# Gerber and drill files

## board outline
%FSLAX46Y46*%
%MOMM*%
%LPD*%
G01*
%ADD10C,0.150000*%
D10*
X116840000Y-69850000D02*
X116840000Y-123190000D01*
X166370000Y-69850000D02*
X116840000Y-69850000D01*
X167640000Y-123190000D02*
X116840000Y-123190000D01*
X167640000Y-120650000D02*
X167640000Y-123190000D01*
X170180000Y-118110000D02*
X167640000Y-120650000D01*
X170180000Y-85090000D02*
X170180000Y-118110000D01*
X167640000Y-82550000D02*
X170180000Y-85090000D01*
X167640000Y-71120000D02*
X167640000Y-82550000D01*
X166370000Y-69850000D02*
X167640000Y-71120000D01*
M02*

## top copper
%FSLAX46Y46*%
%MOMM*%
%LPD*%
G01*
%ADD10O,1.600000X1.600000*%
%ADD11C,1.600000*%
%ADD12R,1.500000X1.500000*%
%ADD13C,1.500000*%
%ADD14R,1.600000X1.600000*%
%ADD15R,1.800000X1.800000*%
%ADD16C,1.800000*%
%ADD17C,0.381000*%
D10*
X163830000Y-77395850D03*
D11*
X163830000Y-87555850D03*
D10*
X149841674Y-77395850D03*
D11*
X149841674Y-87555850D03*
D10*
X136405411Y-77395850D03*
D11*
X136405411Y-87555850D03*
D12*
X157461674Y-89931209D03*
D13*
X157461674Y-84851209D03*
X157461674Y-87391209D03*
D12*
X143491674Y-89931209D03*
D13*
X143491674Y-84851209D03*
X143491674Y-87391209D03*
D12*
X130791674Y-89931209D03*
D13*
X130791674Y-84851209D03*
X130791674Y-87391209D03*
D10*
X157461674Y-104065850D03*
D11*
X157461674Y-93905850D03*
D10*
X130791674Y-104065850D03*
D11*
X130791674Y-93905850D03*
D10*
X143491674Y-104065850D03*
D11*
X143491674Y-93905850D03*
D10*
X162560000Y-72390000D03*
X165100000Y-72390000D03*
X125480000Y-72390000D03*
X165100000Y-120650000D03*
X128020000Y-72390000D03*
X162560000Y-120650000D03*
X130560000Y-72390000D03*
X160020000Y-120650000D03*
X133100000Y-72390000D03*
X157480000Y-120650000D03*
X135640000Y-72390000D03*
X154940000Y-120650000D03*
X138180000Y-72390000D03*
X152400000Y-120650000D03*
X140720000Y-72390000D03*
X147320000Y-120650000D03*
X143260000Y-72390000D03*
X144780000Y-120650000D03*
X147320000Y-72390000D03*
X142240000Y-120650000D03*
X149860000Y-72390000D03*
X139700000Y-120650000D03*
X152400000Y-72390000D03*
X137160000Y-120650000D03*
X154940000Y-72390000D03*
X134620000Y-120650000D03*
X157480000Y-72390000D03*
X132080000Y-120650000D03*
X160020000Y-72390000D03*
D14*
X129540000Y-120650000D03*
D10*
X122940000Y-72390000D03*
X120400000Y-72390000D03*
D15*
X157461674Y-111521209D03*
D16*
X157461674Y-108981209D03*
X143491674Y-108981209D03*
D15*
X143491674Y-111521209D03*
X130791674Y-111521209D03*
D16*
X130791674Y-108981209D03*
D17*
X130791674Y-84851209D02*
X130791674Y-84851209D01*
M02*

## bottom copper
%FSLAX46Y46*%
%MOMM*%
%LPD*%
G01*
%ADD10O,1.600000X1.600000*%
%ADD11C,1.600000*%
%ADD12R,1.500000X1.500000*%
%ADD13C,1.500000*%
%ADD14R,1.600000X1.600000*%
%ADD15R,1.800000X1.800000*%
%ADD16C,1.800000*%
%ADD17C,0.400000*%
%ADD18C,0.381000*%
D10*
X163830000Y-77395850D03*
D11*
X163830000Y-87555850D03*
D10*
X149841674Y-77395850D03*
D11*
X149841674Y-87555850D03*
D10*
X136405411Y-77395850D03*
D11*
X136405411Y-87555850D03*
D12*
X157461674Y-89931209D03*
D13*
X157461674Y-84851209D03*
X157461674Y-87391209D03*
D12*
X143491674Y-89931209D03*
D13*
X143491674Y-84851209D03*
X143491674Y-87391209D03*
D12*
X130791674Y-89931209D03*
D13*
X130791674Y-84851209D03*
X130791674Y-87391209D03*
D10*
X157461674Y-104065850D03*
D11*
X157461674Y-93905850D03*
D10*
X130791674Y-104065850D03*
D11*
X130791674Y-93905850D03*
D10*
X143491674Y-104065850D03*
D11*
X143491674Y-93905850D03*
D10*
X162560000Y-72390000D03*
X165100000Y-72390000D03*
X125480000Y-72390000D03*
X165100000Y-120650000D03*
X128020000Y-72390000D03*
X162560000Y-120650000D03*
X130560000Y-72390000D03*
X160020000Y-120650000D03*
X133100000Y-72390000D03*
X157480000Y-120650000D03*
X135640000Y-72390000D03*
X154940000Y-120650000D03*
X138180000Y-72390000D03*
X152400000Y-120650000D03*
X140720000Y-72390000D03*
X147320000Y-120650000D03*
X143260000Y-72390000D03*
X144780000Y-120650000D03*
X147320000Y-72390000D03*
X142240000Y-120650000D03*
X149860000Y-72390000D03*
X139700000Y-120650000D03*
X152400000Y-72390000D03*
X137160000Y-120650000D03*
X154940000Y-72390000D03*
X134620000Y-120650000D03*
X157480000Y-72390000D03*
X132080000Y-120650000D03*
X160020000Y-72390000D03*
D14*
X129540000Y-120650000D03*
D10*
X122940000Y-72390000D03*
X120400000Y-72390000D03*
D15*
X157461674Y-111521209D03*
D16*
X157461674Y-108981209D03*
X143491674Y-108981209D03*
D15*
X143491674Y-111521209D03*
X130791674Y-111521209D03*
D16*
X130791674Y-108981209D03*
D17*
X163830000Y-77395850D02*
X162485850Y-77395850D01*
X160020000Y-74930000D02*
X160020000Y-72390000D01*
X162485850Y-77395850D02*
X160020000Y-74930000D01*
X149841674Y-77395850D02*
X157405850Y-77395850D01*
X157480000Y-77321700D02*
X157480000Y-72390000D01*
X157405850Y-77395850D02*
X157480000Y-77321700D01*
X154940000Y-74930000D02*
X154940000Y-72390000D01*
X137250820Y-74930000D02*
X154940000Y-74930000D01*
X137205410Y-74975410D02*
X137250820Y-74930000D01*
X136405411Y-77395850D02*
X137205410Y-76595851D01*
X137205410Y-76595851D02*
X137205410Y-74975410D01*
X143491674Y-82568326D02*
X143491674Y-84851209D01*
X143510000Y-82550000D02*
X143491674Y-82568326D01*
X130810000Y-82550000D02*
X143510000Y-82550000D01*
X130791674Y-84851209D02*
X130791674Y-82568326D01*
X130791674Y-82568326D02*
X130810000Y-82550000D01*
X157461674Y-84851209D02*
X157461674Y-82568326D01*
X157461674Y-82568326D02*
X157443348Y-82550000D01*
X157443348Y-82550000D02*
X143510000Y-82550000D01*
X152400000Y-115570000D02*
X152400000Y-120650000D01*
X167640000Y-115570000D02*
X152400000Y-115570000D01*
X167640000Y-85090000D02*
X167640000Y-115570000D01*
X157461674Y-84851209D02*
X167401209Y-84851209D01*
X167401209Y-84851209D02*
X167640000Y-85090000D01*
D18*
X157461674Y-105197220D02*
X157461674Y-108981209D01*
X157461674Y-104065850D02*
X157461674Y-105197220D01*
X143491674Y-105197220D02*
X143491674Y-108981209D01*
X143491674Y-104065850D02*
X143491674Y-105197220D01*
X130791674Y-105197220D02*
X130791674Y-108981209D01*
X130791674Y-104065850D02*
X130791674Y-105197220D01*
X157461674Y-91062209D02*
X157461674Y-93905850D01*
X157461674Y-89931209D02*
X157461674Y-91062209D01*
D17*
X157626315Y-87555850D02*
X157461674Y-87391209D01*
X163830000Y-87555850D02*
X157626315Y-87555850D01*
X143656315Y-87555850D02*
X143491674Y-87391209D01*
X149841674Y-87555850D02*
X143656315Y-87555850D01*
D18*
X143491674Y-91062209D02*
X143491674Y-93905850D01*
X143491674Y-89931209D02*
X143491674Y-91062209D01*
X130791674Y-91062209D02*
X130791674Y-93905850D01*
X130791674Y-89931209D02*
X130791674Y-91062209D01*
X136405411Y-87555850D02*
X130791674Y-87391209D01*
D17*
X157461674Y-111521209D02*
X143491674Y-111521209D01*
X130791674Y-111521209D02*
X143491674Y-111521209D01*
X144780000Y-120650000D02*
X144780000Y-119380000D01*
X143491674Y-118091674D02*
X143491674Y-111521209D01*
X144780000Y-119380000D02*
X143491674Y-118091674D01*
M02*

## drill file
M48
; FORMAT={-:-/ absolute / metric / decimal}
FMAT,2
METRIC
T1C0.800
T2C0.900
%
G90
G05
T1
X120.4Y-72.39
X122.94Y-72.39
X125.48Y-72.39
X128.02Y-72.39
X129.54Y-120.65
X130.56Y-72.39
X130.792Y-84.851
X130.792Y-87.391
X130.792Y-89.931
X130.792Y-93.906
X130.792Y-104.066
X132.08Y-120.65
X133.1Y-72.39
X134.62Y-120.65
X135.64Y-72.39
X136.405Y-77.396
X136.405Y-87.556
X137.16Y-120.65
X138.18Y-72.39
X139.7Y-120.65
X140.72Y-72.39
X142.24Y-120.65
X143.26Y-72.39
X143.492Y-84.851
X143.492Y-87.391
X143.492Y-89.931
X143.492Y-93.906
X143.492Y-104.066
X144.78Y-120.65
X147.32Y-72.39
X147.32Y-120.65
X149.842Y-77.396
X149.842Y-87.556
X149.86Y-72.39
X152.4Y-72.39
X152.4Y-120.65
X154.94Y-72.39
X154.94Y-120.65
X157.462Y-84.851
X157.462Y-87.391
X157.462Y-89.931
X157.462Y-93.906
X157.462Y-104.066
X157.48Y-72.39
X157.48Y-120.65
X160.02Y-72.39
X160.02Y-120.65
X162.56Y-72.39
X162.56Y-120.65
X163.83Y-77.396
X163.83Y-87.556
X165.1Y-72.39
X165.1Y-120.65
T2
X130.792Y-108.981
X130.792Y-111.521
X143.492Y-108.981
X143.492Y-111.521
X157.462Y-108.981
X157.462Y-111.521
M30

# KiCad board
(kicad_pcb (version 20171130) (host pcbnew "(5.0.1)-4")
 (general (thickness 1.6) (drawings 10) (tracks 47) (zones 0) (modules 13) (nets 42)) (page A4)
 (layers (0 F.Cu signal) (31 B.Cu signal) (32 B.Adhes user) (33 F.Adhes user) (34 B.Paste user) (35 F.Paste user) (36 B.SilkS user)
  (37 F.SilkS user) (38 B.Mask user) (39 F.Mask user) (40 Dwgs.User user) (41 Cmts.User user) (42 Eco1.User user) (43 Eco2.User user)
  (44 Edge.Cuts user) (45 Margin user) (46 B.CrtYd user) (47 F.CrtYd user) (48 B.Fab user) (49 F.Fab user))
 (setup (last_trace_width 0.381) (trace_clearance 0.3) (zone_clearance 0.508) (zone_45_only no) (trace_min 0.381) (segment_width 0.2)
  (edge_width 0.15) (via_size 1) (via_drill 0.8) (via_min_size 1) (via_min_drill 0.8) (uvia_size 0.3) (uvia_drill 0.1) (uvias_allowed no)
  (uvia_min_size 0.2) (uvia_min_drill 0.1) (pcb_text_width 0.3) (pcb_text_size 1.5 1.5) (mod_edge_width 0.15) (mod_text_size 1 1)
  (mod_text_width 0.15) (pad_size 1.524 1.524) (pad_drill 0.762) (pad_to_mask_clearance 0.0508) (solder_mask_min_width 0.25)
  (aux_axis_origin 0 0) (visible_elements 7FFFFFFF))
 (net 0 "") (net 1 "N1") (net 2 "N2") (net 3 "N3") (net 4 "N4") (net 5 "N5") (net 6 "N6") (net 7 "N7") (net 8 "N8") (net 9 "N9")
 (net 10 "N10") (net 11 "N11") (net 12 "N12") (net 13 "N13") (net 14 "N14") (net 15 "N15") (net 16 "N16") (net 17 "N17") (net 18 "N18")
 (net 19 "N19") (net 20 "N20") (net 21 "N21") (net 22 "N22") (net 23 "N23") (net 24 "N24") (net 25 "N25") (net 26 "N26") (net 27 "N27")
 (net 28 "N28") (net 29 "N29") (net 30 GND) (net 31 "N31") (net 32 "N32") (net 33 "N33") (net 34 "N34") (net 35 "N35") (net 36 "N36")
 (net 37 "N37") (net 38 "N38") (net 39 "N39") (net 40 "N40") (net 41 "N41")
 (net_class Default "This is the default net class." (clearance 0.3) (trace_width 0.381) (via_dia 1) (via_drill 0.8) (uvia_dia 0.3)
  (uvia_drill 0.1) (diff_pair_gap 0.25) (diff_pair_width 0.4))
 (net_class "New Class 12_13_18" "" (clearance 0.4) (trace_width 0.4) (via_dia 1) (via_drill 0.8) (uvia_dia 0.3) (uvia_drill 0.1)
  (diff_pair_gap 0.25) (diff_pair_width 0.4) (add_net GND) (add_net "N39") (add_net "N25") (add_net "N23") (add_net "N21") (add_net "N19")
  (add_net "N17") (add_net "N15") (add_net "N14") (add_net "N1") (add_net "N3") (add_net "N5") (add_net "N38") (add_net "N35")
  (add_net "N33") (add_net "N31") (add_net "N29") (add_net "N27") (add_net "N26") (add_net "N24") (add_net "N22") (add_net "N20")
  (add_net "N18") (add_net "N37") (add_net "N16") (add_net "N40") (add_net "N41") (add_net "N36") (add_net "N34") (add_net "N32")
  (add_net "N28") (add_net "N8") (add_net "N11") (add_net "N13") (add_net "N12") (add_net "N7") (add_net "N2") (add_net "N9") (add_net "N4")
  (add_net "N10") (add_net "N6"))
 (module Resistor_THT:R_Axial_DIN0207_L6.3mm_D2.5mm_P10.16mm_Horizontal (layer F.Cu) (at 163.83 87.55585 90)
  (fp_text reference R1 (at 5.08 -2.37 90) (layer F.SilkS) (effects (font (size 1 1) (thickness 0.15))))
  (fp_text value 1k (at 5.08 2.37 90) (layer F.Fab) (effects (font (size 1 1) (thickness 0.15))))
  (pad 2 thru_hole oval (at 10.16 0 90) (size 1.6 1.6) (drill 0.8) (layers *.Cu *.Mask) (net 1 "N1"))
  (pad 1 thru_hole circle (at 0 0 90) (size 1.6 1.6) (drill 0.8) (layers *.Cu *.Mask) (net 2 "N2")))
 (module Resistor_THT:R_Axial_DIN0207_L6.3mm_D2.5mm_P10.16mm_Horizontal (layer F.Cu) (at 149.841674 87.55585 90)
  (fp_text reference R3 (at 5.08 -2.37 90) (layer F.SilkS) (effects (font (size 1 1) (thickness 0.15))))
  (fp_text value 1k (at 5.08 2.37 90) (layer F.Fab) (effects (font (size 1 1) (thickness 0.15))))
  (pad 2 thru_hole oval (at 10.16 0 90) (size 1.6 1.6) (drill 0.8) (layers *.Cu *.Mask) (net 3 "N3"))
  (pad 1 thru_hole circle (at 0 0 90) (size 1.6 1.6) (drill 0.8) (layers *.Cu *.Mask) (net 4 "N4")))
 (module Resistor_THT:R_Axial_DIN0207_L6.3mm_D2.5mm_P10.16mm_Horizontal (layer F.Cu) (at 136.405411 87.55585 90)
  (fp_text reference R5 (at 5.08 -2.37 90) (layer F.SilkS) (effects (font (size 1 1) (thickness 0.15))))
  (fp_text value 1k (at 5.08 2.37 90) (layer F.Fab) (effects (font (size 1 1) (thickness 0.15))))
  (pad 2 thru_hole oval (at 10.16 0 90) (size 1.6 1.6) (drill 0.8) (layers *.Cu *.Mask) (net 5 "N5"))
  (pad 1 thru_hole circle (at 0 0 90) (size 1.6 1.6) (drill 0.8) (layers *.Cu *.Mask) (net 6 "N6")))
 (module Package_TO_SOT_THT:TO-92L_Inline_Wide (layer F.Cu) (at 157.461674 89.931209 90)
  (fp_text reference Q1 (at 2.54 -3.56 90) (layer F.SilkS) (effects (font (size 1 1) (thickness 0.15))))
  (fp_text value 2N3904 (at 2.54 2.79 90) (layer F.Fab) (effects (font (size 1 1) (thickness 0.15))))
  (pad 1 thru_hole rect (at 0 0 180) (size 1.5 1.5) (drill 0.8) (layers *.Cu *.Mask) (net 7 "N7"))
  (pad 3 thru_hole circle (at 5.08 0 180) (size 1.5 1.5) (drill 0.8) (layers *.Cu *.Mask) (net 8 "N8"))
  (pad 2 thru_hole circle (at 2.54 0 180) (size 1.5 1.5) (drill 0.8) (layers *.Cu *.Mask) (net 2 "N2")))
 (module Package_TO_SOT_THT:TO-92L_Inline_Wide (layer F.Cu) (at 143.491674 89.931209 90)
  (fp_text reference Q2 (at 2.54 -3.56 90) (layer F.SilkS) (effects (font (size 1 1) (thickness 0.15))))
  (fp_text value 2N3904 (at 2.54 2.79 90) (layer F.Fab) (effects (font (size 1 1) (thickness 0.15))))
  (pad 1 thru_hole rect (at 0 0 180) (size 1.5 1.5) (drill 0.8) (layers *.Cu *.Mask) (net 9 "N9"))
  (pad 3 thru_hole circle (at 5.08 0 180) (size 1.5 1.5) (drill 0.8) (layers *.Cu *.Mask) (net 8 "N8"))
  (pad 2 thru_hole circle (at 2.54 0 180) (size 1.5 1.5) (drill 0.8) (layers *.Cu *.Mask) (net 4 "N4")))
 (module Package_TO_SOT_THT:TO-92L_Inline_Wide (layer F.Cu) (at 130.791674 89.931209 90)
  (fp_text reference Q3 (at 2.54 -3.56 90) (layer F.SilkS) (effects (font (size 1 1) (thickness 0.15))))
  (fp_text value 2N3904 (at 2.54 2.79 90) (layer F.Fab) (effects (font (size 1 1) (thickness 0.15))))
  (pad 1 thru_hole rect (at 0 0 180) (size 1.5 1.5) (drill 0.8) (layers *.Cu *.Mask) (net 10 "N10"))
  (pad 3 thru_hole circle (at 5.08 0 180) (size 1.5 1.5) (drill 0.8) (layers *.Cu *.Mask) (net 8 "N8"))
  (pad 2 thru_hole circle (at 2.54 0 180) (size 1.5 1.5) (drill 0.8) (layers *.Cu *.Mask) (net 6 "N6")))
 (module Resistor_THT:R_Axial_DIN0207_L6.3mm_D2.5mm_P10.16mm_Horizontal (layer F.Cu) (at 157.461674 93.90585 270)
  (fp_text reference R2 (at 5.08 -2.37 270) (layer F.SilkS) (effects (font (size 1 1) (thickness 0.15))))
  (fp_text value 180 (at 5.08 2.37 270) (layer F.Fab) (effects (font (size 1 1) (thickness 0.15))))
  (pad 2 thru_hole oval (at 10.16 0 270) (size 1.6 1.6) (drill 0.8) (layers *.Cu *.Mask) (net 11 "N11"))
  (pad 1 thru_hole circle (at 0 0 270) (size 1.6 1.6) (drill 0.8) (layers *.Cu *.Mask) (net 7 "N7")))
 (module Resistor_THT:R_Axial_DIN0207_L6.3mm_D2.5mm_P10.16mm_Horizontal (layer F.Cu) (at 130.791674 93.90585 270)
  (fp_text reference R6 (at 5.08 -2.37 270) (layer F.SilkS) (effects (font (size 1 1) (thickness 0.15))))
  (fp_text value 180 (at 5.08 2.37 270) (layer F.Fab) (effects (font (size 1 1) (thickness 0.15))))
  (pad 2 thru_hole oval (at 10.16 0 270) (size 1.6 1.6) (drill 0.8) (layers *.Cu *.Mask) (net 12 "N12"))
  (pad 1 thru_hole circle (at 0 0 270) (size 1.6 1.6) (drill 0.8) (layers *.Cu *.Mask) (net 10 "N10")))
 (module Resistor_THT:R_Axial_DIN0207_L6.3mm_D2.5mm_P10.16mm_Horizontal (layer F.Cu) (at 143.491674 93.90585 270)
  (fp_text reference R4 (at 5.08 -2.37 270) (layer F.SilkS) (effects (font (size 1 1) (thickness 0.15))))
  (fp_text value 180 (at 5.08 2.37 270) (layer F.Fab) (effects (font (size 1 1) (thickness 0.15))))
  (pad 2 thru_hole oval (at 10.16 0 270) (size 1.6 1.6) (drill 0.8) (layers *.Cu *.Mask) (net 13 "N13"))
  (pad 1 thru_hole circle (at 0 0 270) (size 1.6 1.6) (drill 0.8) (layers *.Cu *.Mask) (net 9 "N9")))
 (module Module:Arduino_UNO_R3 (layer B.Cu) (at 129.54 120.65)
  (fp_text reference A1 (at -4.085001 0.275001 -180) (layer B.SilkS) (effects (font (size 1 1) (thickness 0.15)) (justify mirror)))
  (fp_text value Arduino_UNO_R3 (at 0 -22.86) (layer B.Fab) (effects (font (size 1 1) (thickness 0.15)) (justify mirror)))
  (pad 16 thru_hole oval (at 33.02 -48.26 270) (size 1.6 1.6) (drill 0.8) (layers *.Cu *.Mask) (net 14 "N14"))
  (pad 15 thru_hole oval (at 35.56 -48.26 270) (size 1.6 1.6) (drill 0.8) (layers *.Cu *.Mask) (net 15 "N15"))
  (pad 30 thru_hole oval (at -4.06 -48.26 270) (size 1.6 1.6) (drill 0.8) (layers *.Cu *.Mask) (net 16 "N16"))
  (pad 14 thru_hole oval (at 35.56 0 270) (size 1.6 1.6) (drill 0.8) (layers *.Cu *.Mask) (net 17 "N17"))
  (pad 29 thru_hole oval (at -1.52 -48.26 270) (size 1.6 1.6) (drill 0.8) (layers *.Cu *.Mask) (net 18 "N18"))
  (pad 13 thru_hole oval (at 33.02 0 270) (size 1.6 1.6) (drill 0.8) (layers *.Cu *.Mask) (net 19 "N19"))
  (pad 28 thru_hole oval (at 1.02 -48.26 270) (size 1.6 1.6) (drill 0.8) (layers *.Cu *.Mask) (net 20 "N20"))
  (pad 12 thru_hole oval (at 30.48 0 270) (size 1.6 1.6) (drill 0.8) (layers *.Cu *.Mask) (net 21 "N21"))
  (pad 27 thru_hole oval (at 3.56 -48.26 270) (size 1.6 1.6) (drill 0.8) (layers *.Cu *.Mask) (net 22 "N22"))
  (pad 11 thru_hole oval (at 27.94 0 270) (size 1.6 1.6) (drill 0.8) (layers *.Cu *.Mask) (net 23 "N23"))
  (pad 26 thru_hole oval (at 6.1 -48.26 270) (size 1.6 1.6) (drill 0.8) (layers *.Cu *.Mask) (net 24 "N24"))
  (pad 10 thru_hole oval (at 25.4 0 270) (size 1.6 1.6) (drill 0.8) (layers *.Cu *.Mask) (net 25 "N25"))
  (pad 25 thru_hole oval (at 8.64 -48.26 270) (size 1.6 1.6) (drill 0.8) (layers *.Cu *.Mask) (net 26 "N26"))
  (pad 9 thru_hole oval (at 22.86 0 270) (size 1.6 1.6) (drill 0.8) (layers *.Cu *.Mask) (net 8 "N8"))
  (pad 24 thru_hole oval (at 11.18 -48.26 270) (size 1.6 1.6) (drill 0.8) (layers *.Cu *.Mask) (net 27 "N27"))
  (pad 8 thru_hole oval (at 17.78 0 270) (size 1.6 1.6) (drill 0.8) (layers *.Cu *.Mask) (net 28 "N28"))
  (pad 23 thru_hole oval (at 13.72 -48.26 270) (size 1.6 1.6) (drill 0.8) (layers *.Cu *.Mask) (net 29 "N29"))
  (pad 7 thru_hole oval (at 15.24 0 270) (size 1.6 1.6) (drill 0.8) (layers *.Cu *.Mask) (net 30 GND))
  (pad 22 thru_hole oval (at 17.78 -48.26 270) (size 1.6 1.6) (drill 0.8) (layers *.Cu *.Mask) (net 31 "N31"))
  (pad 6 thru_hole oval (at 12.7 0 270) (size 1.6 1.6) (drill 0.8) (layers *.Cu *.Mask) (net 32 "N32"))
  (pad 21 thru_hole oval (at 20.32 -48.26 270) (size 1.6 1.6) (drill 0.8) (layers *.Cu *.Mask) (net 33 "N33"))
  (pad 5 thru_hole oval (at 10.16 0 270) (size 1.6 1.6) (drill 0.8) (layers *.Cu *.Mask) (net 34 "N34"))
  (pad 20 thru_hole oval (at 22.86 -48.26 270) (size 1.6 1.6) (drill 0.8) (layers *.Cu *.Mask) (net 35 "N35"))
  (pad 4 thru_hole oval (at 7.62 0 270) (size 1.6 1.6) (drill 0.8) (layers *.Cu *.Mask) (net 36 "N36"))
  (pad 19 thru_hole oval (at 25.4 -48.26 270) (size 1.6 1.6) (drill 0.8) (layers *.Cu *.Mask) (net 5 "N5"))
  (pad 3 thru_hole oval (at 5.08 0 270) (size 1.6 1.6) (drill 0.8) (layers *.Cu *.Mask) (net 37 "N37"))
  (pad 18 thru_hole oval (at 27.94 -48.26 270) (size 1.6 1.6) (drill 0.8) (layers *.Cu *.Mask) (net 3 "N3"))
  (pad 2 thru_hole oval (at 2.54 0 270) (size 1.6 1.6) (drill 0.8) (layers *.Cu *.Mask) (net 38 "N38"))
  (pad 17 thru_hole oval (at 30.48 -48.26 270) (size 1.6 1.6) (drill 0.8) (layers *.Cu *.Mask) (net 1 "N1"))
  (pad 1 thru_hole rect (at 0 0 270) (size 1.6 1.6) (drill 0.8) (layers *.Cu *.Mask) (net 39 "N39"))
  (pad 31 thru_hole oval (at -6.6 -48.26 270) (size 1.6 1.6) (drill 0.8) (layers *.Cu *.Mask) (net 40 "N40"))
  (pad 32 thru_hole oval (at -9.14 -48.26 270) (size 1.6 1.6) (drill 0.8) (layers *.Cu *.Mask) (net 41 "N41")))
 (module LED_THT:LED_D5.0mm (layer F.Cu) (at 157.461674 111.521209 90)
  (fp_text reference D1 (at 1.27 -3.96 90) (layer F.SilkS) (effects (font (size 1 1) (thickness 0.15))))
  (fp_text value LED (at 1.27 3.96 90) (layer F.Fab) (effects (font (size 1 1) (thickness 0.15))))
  (pad 1 thru_hole rect (at 0 0 90) (size 1.8 1.8) (drill 0.9) (layers *.Cu *.Mask) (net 30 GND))
  (pad 2 thru_hole circle (at 2.54 0 90) (size 1.8 1.8) (drill 0.9) (layers *.Cu *.Mask) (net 11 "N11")))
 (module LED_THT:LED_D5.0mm (layer F.Cu) (at 143.491674 111.521209 90)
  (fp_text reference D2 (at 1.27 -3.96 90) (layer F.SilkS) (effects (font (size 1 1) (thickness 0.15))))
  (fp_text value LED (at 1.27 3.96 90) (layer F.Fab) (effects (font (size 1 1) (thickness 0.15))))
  (pad 2 thru_hole circle (at 2.54 0 90) (size 1.8 1.8) (drill 0.9) (layers *.Cu *.Mask) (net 13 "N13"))
  (pad 1 thru_hole rect (at 0 0 90) (size 1.8 1.8) (drill 0.9) (layers *.Cu *.Mask) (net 30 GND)))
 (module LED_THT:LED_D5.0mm (layer F.Cu) (at 130.791674 111.521209 90)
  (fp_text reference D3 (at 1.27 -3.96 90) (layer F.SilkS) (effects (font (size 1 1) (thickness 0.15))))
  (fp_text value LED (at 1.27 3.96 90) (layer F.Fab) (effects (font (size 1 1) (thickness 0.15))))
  (pad 1 thru_hole rect (at 0 0 90) (size 1.8 1.8) (drill 0.9) (layers *.Cu *.Mask) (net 30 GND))
  (pad 2 thru_hole circle (at 2.54 0 90) (size 1.8 1.8) (drill 0.9) (layers *.Cu *.Mask) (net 12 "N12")))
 (gr_line (start 116.84 69.85) (end 116.84 123.19) (layer Edge.Cuts) (width 0.15))
 (gr_line (start 166.37 69.85) (end 116.84 69.85) (layer Edge.Cuts) (width 0.15))
 (gr_line (start 167.64 123.19) (end 116.84 123.19) (layer Edge.Cuts) (width 0.15))
 (gr_line (start 167.64 120.65) (end 167.64 123.19) (layer Edge.Cuts) (width 0.15))
 (gr_line (start 170.18 118.11) (end 167.64 120.65) (layer Edge.Cuts) (width 0.15))
 (gr_line (start 170.18 85.09) (end 170.18 118.11) (layer Edge.Cuts) (width 0.15))
 (gr_line (start 167.64 82.55) (end 170.18 85.09) (layer Edge.Cuts) (width 0.15))
 (gr_line (start 167.64 71.12) (end 167.64 82.55) (layer Edge.Cuts) (width 0.15))
 (gr_line (start 166.37 69.85) (end 167.64 71.12) (layer Edge.Cuts) (width 0.15))
 (segment (start 163.83 77.39585) (end 162.48585 77.39585) (width 0.4) (layer B.Cu) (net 1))
 (segment (start 160.02 74.93) (end 160.02 72.39) (width 0.4) (layer B.Cu) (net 1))
 (segment (start 162.48585 77.39585) (end 160.02 74.93) (width 0.4) (layer B.Cu) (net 1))
 (segment (start 149.841674 77.39585) (end 157.40585 77.39585) (width 0.4) (layer B.Cu) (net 3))
 (segment (start 157.48 77.3217) (end 157.48 72.39) (width 0.4) (layer B.Cu) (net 3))
 (segment (start 157.40585 77.39585) (end 157.48 77.3217) (width 0.4) (layer B.Cu) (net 3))
 (segment (start 154.94 74.93) (end 154.94 72.39) (width 0.4) (layer B.Cu) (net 5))
 (segment (start 137.25082 74.93) (end 154.94 74.93) (width 0.4) (layer B.Cu) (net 5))
 (segment (start 137.20541 74.97541) (end 137.25082 74.93) (width 0.4) (layer B.Cu) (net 5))
 (segment (start 136.405411 77.39585) (end 137.20541 76.595851) (width 0.4) (layer B.Cu) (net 5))
 (segment (start 137.20541 76.595851) (end 137.20541 74.97541) (width 0.4) (layer B.Cu) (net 5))
 (segment (start 130.791674 84.851209) (end 130.791674 84.851209) (width 0.381) (layer F.Cu) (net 8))
 (segment (start 143.491674 82.568326) (end 143.491674 84.851209) (width 0.4) (layer B.Cu) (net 8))
 (segment (start 143.51 82.55) (end 143.491674 82.568326) (width 0.4) (layer B.Cu) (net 8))
 (segment (start 130.81 82.55) (end 143.51 82.55) (width 0.4) (layer B.Cu) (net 8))
 (segment (start 130.791674 84.851209) (end 130.791674 82.568326) (width 0.4) (layer B.Cu) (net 8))
 (segment (start 130.791674 82.568326) (end 130.81 82.55) (width 0.4) (layer B.Cu) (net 8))
 (segment (start 157.461674 84.851209) (end 157.461674 82.568326) (width 0.4) (layer B.Cu) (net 8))
 (segment (start 157.461674 82.568326) (end 157.443348 82.55) (width 0.4) (layer B.Cu) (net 8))
 (segment (start 157.443348 82.55) (end 143.51 82.55) (width 0.4) (layer B.Cu) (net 8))
 (segment (start 152.4 115.57) (end 152.4 120.65) (width 0.4) (layer B.Cu) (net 8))
 (segment (start 167.64 115.57) (end 152.4 115.57) (width 0.4) (layer B.Cu) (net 8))
 (segment (start 167.64 85.09) (end 167.64 115.57) (width 0.4) (layer B.Cu) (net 8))
 (segment (start 157.461674 84.851209) (end 167.401209 84.851209) (width 0.4) (layer B.Cu) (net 8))
 (segment (start 167.401209 84.851209) (end 167.64 85.09) (width 0.4) (layer B.Cu) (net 8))
 (segment (start 157.461674 105.19722) (end 157.461674 108.981209) (width 0.381) (layer B.Cu) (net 11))
 (segment (start 157.461674 104.06585) (end 157.461674 105.19722) (width 0.381) (layer B.Cu) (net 11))
 (segment (start 143.491674 105.19722) (end 143.491674 108.981209) (width 0.381) (layer B.Cu) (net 13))
 (segment (start 143.491674 104.06585) (end 143.491674 105.19722) (width 0.381) (layer B.Cu) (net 13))
 (segment (start 130.791674 105.19722) (end 130.791674 108.981209) (width 0.381) (layer B.Cu) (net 12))
 (segment (start 130.791674 104.06585) (end 130.791674 105.19722) (width 0.381) (layer B.Cu) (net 12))
 (segment (start 157.461674 91.062209) (end 157.461674 93.90585) (width 0.381) (layer B.Cu) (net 7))
 (segment (start 157.461674 89.931209) (end 157.461674 91.062209) (width 0.381) (layer B.Cu) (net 7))
 (segment (start 157.626315 87.55585) (end 157.461674 87.391209) (width 0.4) (layer B.Cu) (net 2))
 (segment (start 163.83 87.55585) (end 157.626315 87.55585) (width 0.4) (layer B.Cu) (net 2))
 (segment (start 143.656315 87.55585) (end 143.491674 87.391209) (width 0.4) (layer B.Cu) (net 4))
 (segment (start 149.841674 87.55585) (end 143.656315 87.55585) (width 0.4) (layer B.Cu) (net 4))
 (segment (start 143.491674 91.062209) (end 143.491674 93.90585) (width 0.381) (layer B.Cu) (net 9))
 (segment (start 143.491674 89.931209) (end 143.491674 91.062209) (width 0.381) (layer B.Cu) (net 9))
 (segment (start 130.791674 91.062209) (end 130.791674 93.90585) (width 0.381) (layer B.Cu) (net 10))
 (segment (start 130.791674 89.931209) (end 130.791674 91.062209) (width 0.381) (layer B.Cu) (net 10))
 (segment (start 136.405411 87.55585) (end 130.791674 87.391209) (width 0.381) (layer B.Cu) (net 6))
 (segment (start 157.461674 111.521209) (end 143.491674 111.521209) (width 0.4) (layer B.Cu) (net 30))
 (segment (start 130.791674 111.521209) (end 143.491674 111.521209) (width 0.4) (layer B.Cu) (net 30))
 (segment (start 144.78 120.65) (end 144.78 119.38) (width 0.4) (layer B.Cu) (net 30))
 (segment (start 143.491674 118.091674) (end 143.491674 111.521209) (width 0.4) (layer B.Cu) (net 30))
 (segment (start 144.78 119.38) (end 143.491674 118.091674) (width 0.4) (layer B.Cu) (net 30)))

